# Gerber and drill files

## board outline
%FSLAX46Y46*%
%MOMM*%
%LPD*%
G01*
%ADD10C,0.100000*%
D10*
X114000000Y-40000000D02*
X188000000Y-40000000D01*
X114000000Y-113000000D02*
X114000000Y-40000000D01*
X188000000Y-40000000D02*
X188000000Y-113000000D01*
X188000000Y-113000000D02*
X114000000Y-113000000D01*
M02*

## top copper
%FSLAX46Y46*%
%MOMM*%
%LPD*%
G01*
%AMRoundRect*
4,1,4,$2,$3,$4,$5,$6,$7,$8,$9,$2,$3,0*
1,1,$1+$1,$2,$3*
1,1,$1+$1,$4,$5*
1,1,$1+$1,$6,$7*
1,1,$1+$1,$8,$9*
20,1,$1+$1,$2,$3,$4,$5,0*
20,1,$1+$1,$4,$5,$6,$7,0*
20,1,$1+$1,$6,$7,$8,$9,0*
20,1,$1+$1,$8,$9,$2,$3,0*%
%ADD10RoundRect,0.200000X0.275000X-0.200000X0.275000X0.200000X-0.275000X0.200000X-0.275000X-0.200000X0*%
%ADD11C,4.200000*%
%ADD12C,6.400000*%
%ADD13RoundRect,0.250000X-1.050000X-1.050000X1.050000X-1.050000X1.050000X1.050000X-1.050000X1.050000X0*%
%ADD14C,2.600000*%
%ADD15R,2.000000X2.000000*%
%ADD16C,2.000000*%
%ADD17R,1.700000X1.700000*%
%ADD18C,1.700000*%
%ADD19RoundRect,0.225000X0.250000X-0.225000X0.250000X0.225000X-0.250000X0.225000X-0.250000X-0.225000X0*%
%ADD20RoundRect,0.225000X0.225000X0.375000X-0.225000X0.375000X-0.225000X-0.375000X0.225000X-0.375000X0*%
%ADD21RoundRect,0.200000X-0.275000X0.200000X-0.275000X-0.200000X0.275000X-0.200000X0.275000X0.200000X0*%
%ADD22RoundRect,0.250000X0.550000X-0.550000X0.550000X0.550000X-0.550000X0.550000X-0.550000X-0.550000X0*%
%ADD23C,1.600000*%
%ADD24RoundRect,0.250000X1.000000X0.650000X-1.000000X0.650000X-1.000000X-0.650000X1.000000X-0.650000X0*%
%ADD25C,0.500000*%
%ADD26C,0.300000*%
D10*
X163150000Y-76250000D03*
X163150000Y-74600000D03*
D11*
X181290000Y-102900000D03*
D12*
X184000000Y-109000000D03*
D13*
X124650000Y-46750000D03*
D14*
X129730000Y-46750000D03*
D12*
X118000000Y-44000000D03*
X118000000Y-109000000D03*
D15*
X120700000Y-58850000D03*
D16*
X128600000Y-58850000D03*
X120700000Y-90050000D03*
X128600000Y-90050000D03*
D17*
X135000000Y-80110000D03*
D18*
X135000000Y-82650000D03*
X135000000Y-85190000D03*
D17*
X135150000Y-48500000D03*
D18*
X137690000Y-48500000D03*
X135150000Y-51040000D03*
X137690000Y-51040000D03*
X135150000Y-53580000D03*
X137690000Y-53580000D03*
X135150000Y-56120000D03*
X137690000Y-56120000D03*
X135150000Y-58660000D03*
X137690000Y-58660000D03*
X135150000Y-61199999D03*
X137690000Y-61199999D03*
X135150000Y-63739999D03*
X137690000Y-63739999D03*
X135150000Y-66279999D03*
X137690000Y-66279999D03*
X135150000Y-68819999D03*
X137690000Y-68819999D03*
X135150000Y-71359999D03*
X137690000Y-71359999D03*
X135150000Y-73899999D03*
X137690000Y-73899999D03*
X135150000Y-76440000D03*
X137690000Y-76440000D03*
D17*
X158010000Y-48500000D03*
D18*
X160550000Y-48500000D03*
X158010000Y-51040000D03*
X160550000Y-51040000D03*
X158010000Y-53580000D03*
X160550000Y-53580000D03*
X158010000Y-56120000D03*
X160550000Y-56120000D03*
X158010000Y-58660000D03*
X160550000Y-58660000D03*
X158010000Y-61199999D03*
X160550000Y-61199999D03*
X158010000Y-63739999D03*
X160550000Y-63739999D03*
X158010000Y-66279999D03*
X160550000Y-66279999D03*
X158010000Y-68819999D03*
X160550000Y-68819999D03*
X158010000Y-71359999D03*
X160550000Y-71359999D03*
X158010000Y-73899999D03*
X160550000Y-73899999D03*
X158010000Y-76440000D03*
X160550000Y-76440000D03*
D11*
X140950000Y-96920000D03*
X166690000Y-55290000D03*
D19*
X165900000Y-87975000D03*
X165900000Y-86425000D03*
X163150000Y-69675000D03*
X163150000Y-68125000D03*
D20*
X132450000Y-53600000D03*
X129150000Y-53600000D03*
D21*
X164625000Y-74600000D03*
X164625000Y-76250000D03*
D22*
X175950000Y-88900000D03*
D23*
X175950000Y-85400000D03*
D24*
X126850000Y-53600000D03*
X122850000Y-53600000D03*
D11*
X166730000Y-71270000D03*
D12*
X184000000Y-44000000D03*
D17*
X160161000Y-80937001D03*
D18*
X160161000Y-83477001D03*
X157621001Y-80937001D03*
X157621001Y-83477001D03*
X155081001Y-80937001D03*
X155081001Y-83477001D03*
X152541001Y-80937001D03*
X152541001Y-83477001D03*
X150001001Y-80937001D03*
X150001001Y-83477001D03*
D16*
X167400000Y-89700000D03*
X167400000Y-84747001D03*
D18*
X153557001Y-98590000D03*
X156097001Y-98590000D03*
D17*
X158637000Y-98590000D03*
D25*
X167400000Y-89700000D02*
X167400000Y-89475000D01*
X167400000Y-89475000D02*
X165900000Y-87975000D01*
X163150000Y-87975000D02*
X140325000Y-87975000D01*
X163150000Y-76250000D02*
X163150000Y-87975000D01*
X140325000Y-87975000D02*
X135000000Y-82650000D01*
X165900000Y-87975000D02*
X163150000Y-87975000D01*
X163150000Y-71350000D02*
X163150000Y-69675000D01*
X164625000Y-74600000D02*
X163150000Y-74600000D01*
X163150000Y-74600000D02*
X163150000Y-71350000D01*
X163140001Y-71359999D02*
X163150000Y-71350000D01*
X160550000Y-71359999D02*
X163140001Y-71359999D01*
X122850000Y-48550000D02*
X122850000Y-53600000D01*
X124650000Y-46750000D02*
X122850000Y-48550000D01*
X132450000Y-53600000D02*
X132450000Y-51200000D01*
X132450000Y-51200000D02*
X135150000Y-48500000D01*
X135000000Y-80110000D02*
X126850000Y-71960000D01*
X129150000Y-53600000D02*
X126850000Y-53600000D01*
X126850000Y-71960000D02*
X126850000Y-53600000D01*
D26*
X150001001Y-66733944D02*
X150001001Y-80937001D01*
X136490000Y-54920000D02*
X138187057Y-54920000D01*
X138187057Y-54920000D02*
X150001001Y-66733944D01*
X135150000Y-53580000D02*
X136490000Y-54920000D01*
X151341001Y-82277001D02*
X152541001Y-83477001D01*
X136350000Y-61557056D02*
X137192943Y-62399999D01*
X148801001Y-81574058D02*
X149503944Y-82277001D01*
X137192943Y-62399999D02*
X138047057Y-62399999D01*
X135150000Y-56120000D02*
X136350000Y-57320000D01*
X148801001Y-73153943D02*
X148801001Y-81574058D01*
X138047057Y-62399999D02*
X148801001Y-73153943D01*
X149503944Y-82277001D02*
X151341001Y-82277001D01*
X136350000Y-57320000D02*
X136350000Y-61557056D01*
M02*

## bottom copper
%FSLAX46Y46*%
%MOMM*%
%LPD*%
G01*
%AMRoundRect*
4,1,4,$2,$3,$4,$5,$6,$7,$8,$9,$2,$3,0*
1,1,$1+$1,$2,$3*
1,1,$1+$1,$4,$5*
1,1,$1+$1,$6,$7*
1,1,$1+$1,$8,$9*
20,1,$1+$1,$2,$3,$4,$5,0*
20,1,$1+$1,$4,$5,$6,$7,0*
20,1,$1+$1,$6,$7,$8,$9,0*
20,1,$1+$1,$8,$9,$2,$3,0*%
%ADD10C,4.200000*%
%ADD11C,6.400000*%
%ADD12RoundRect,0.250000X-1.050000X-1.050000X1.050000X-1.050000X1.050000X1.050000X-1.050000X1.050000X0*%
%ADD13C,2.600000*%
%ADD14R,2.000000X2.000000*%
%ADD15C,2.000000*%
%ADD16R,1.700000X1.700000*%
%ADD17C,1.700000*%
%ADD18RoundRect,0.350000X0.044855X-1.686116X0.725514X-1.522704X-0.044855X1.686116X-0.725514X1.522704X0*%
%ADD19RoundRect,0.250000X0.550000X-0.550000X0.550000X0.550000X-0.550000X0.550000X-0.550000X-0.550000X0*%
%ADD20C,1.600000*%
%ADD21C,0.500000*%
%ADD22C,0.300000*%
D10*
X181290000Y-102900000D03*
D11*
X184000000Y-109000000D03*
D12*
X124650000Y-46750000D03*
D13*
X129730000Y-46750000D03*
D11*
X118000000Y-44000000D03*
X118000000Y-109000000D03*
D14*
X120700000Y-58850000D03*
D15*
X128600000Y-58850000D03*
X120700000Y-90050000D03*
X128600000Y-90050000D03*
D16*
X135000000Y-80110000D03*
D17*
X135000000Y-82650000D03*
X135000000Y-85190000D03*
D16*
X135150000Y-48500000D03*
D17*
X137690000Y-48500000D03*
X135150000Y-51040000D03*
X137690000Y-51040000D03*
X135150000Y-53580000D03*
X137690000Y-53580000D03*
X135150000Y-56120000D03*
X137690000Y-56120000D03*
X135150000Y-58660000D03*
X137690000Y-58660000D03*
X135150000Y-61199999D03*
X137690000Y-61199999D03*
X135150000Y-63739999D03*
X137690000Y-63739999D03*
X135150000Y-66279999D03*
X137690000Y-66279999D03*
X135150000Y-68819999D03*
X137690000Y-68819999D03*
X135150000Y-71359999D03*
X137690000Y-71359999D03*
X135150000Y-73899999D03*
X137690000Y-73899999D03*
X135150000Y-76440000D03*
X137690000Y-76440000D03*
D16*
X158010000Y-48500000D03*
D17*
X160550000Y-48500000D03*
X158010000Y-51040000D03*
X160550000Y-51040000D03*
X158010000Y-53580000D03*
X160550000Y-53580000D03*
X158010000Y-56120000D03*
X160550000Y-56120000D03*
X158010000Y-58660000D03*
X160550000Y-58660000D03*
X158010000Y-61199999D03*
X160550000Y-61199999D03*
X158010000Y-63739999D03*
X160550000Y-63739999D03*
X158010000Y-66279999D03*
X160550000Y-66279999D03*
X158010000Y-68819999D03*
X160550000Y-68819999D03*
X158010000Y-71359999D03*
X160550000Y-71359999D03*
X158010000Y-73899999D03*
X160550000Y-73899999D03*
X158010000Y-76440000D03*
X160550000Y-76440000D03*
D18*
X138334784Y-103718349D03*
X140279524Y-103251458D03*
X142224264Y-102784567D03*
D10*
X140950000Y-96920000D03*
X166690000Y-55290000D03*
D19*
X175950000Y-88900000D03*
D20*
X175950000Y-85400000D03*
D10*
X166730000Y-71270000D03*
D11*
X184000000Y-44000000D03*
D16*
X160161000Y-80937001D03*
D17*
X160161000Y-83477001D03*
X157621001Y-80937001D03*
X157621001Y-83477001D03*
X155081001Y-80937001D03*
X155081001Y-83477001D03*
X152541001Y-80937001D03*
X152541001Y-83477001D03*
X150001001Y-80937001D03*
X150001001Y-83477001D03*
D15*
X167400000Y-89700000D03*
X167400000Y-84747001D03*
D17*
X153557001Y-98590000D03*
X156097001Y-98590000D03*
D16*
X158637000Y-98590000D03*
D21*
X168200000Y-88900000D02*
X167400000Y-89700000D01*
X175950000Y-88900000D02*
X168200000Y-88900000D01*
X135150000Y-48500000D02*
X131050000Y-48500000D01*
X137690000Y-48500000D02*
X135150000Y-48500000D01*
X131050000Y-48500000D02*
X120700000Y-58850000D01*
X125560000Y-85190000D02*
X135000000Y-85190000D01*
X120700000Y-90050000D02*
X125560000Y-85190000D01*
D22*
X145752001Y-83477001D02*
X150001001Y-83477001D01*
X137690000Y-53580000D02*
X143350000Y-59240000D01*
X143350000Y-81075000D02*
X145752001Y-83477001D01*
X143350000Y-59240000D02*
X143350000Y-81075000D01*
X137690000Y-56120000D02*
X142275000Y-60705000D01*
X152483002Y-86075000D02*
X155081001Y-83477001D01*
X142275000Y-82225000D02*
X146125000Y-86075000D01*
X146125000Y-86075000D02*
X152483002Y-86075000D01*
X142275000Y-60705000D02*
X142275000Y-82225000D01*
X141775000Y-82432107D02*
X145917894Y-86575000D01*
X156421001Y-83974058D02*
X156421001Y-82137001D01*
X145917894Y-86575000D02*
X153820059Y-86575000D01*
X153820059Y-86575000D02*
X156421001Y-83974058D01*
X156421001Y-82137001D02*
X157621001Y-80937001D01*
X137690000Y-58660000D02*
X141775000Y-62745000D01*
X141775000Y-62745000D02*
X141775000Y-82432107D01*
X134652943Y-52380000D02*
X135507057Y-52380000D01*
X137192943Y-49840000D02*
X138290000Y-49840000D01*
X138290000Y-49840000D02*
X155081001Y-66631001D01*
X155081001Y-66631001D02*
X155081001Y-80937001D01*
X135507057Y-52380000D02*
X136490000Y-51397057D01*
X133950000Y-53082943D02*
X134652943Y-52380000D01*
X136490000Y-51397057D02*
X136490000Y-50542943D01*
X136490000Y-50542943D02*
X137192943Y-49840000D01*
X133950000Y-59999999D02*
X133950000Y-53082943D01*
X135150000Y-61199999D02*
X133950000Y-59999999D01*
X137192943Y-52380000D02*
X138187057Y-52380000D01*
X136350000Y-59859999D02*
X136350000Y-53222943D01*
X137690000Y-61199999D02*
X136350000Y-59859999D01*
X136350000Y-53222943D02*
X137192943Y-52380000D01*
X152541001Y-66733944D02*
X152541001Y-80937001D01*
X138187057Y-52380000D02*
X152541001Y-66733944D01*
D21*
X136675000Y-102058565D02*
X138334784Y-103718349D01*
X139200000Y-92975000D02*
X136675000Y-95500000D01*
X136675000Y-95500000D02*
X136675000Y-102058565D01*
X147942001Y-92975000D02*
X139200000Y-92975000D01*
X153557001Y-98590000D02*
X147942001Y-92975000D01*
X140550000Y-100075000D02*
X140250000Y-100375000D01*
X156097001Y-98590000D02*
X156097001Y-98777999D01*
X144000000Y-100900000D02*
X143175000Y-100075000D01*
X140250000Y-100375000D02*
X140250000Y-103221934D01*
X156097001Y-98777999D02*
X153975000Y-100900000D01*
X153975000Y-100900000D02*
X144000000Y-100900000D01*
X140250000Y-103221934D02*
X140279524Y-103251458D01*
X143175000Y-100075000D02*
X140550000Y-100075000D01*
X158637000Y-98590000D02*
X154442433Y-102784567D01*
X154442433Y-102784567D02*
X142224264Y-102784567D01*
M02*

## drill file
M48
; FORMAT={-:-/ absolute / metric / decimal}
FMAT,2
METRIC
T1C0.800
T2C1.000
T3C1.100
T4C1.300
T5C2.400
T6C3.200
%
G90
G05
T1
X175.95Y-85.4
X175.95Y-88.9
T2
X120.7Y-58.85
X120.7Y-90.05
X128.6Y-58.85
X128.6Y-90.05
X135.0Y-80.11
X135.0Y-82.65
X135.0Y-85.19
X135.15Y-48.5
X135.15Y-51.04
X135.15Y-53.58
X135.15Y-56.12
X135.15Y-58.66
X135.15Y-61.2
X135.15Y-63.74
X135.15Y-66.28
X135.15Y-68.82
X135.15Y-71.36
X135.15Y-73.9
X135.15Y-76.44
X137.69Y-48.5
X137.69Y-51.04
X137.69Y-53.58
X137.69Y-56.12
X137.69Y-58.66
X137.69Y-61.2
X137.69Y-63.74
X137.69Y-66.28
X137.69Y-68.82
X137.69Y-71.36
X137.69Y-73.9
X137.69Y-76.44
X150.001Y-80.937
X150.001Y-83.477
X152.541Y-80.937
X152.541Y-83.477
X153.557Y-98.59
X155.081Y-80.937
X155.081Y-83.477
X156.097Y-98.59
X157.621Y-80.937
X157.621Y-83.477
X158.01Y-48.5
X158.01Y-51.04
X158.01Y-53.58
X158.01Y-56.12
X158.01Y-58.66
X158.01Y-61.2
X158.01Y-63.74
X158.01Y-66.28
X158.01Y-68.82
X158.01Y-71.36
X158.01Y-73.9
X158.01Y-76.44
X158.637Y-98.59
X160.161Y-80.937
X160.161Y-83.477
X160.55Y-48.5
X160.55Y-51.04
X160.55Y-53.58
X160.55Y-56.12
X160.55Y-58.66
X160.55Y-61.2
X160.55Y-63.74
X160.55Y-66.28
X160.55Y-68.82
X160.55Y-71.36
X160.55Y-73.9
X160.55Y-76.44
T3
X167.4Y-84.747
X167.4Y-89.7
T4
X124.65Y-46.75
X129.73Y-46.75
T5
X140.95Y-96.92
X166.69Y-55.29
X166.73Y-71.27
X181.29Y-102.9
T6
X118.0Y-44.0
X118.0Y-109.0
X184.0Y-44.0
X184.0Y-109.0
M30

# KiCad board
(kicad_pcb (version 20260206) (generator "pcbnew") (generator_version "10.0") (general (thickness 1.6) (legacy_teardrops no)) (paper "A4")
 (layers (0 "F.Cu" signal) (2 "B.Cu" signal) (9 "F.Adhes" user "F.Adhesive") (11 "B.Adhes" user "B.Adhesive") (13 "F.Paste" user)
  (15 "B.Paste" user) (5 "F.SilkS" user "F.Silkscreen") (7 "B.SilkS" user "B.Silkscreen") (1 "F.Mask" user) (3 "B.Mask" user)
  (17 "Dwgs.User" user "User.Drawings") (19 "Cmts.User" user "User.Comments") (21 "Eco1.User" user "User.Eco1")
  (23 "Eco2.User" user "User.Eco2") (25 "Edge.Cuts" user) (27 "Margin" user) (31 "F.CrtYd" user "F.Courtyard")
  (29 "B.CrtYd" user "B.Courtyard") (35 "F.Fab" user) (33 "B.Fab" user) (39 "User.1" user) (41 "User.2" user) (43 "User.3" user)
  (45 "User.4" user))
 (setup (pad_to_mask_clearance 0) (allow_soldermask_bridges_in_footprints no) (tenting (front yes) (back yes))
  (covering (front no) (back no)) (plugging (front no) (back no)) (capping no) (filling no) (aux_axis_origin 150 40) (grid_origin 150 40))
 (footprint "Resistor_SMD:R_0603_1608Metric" (layer "F.Cu") (at 163.15 75.425 90)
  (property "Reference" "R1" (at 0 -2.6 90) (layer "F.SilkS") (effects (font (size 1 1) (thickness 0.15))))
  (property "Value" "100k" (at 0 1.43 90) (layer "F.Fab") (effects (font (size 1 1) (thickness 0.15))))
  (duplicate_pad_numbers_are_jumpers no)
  (pad "1" smd roundrect (at -0.825 0 90) (size 0.8 0.95) (layers "F.Cu" "F.Mask" "F.Paste") (roundrect_rratio 0.25) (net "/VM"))
  (pad "2" smd roundrect (at 0.825 0 90) (size 0.8 0.95) (layers "F.Cu" "F.Mask" "F.Paste") (roundrect_rratio 0.25) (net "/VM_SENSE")))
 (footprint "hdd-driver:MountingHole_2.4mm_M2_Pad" (layer "F.Cu") (at 181.29 102.9)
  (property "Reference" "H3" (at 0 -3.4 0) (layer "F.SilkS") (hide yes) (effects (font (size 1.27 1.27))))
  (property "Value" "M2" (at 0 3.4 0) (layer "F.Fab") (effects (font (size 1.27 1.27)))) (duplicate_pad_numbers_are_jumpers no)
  (pad "1" thru_hole circle (at 0 0) (size 4.2 4.2) (drill 2.4) (layers "*.Cu" "*.Mask") (remove_unused_layers no) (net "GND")))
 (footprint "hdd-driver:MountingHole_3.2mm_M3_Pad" (layer "F.Cu") (at 184 109)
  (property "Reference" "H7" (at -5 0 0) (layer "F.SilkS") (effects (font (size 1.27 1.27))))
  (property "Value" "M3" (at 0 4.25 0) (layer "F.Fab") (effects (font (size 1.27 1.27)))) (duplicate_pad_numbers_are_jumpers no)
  (pad "1" thru_hole circle (at 0 0) (size 6.4 6.4) (drill 3.2) (layers "*.Cu" "*.Mask") (remove_unused_layers no) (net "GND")))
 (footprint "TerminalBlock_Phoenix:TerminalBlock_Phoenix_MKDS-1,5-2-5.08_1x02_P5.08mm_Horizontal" (layer "F.Cu") (at 124.65 46.75)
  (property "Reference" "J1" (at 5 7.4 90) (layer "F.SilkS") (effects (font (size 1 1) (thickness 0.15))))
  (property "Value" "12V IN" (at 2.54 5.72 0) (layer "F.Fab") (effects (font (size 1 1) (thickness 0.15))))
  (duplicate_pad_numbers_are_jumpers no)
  (pad "1" thru_hole roundrect (at 0 0) (size 2.6 2.6) (drill 1.3) (layers "*.Cu" "*.Mask") (remove_unused_layers no)
   (roundrect_rratio 0.096154) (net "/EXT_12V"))
  (pad "2" thru_hole circle (at 5.08 0) (size 2.6 2.6) (drill 1.3) (layers "*.Cu" "*.Mask") (remove_unused_layers no) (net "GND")))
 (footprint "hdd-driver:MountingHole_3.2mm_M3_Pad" (layer "F.Cu") (at 118 44)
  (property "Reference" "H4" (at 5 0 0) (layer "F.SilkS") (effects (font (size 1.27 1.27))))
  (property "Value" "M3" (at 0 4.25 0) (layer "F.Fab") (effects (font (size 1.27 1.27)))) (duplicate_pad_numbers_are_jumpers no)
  (pad "1" thru_hole circle (at 0 0) (size 6.4 6.4) (drill 3.2) (layers "*.Cu" "*.Mask") (remove_unused_layers no) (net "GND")))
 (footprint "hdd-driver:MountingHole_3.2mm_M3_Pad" (layer "F.Cu") (at 118 109)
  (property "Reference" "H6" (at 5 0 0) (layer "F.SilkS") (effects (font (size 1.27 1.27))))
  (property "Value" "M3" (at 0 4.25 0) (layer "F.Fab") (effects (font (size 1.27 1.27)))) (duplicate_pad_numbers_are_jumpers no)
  (pad "1" thru_hole circle (at 0 0) (size 6.4 6.4) (drill 3.2) (layers "*.Cu" "*.Mask") (remove_unused_layers no) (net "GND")))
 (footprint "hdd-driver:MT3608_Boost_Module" (layer "F.Cu") (at 124.1 74.45 -90)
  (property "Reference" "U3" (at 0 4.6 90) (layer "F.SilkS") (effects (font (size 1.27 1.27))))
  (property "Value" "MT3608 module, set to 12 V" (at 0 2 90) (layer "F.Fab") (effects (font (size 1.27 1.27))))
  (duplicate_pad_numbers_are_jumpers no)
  (pad "1" thru_hole rect (at -15.6 3.4 270) (size 2 2) (drill 1) (layers "*.Cu" "*.Mask") (remove_unused_layers no) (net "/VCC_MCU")
   (thermal_bridge_angle 45))
  (pad "2" thru_hole circle (at -15.6 -4.5 270) (size 2 2) (drill 1) (layers "*.Cu" "*.Mask") (remove_unused_layers no) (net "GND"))
  (pad "3" thru_hole circle (at 15.6 3.4 270) (size 2 2) (drill 1) (layers "*.Cu" "*.Mask") (remove_unused_layers no) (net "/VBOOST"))
  (pad "4" thru_hole circle (at 15.6 -4.5 270) (size 2 2) (drill 1) (layers "*.Cu" "*.Mask") (remove_unused_layers no) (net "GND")))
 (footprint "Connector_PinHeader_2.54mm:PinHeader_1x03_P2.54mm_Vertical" (layer "F.Cu") (at 135 80.11)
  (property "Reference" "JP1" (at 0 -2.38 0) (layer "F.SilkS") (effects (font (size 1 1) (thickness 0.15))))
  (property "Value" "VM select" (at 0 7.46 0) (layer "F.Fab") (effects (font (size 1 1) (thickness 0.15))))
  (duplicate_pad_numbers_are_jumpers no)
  (pad "1" thru_hole rect (at 0 0) (size 1.7 1.7) (drill 1) (layers "*.Cu" "*.Mask") (remove_unused_layers no) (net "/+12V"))
  (pad "2" thru_hole circle (at 0 2.54) (size 1.7 1.7) (drill 1) (layers "*.Cu" "*.Mask") (remove_unused_layers no) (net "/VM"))
  (pad "3" thru_hole circle (at 0 5.08) (size 1.7 1.7) (drill 1) (layers "*.Cu" "*.Mask") (remove_unused_layers no) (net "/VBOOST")))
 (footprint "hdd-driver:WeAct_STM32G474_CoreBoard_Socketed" (layer "F.Cu") (at 147.85 59.67 -90)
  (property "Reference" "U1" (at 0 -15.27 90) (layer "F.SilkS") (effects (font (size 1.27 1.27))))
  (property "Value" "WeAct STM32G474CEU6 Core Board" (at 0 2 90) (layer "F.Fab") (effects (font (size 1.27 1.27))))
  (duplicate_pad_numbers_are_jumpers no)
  (pad "P1.1" thru_hole rect (at -11.17 12.7 270) (size 1.7 1.7) (drill 1) (layers "*.Cu" "*.Mask") (remove_unused_layers no)
   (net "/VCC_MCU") (thermal_bridge_angle 45))
  (pad "P1.2" thru_hole circle (at -11.17 10.16 270) (size 1.7 1.7) (drill 1) (layers "*.Cu" "*.Mask") (remove_unused_layers no)
   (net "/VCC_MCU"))
  (pad "P1.3" thru_hole circle (at -8.63 12.7 270) (size 1.7 1.7) (drill 1) (layers "*.Cu" "*.Mask") (remove_unused_layers no) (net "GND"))
  (pad "P1.4" thru_hole circle (at -8.63 10.16 270) (size 1.7 1.7) (drill 1) (layers "*.Cu" "*.Mask") (remove_unused_layers no) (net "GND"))
  (pad "P1.5" thru_hole circle (at -6.09 12.7 270) (size 1.7 1.7) (drill 1) (layers "*.Cu" "*.Mask") (remove_unused_layers no)
   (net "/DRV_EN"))
  (pad "P1.6" thru_hole circle (at -6.09 10.16 270) (size 1.7 1.7) (drill 1) (layers "*.Cu" "*.Mask") (remove_unused_layers no)
   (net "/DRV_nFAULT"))
  (pad "P1.7" thru_hole circle (at -3.55 12.7 270) (size 1.7 1.7) (drill 1) (layers "*.Cu" "*.Mask") (remove_unused_layers no)
   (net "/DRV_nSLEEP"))
  (pad "P1.8" thru_hole circle (at -3.55 10.16 270) (size 1.7 1.7) (drill 1) (layers "*.Cu" "*.Mask") (remove_unused_layers no)
   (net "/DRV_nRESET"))
  (pad "P1.9" thru_hole circle (at -1.01 12.7 270) (size 1.7 1.7) (drill 1) (layers "*.Cu" "*.Mask") (remove_unused_layers no)
   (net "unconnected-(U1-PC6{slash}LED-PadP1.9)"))
  (pad "P1.10" thru_hole circle (at -1.01 10.16 270) (size 1.7 1.7) (drill 1) (layers "*.Cu" "*.Mask") (remove_unused_layers no)
   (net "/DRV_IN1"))
  (pad "P1.11" thru_hole circle (at 1.529999 12.7 270) (size 1.7 1.7) (drill 1) (layers "*.Cu" "*.Mask") (remove_unused_layers no)
   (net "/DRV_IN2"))
  (pad "P1.12" thru_hole circle (at 1.529999 10.16 270) (size 1.7 1.7) (drill 1) (layers "*.Cu" "*.Mask") (remove_unused_layers no)
   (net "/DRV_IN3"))
  (pad "P1.13" thru_hole circle (at 4.069999 12.7 270) (size 1.7 1.7) (drill 1) (layers "*.Cu" "*.Mask") (remove_unused_layers no)
   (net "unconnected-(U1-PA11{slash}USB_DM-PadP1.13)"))
  (pad "P1.14" thru_hole circle (at 4.069999 10.16 270) (size 1.7 1.7) (drill 1) (layers "*.Cu" "*.Mask") (remove_unused_layers no)
   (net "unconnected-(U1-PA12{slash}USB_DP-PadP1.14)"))
  (pad "P1.15" thru_hole circle (at 6.609999 12.7 270) (size 1.7 1.7) (drill 1) (layers "*.Cu" "*.Mask") (remove_unused_layers no)
   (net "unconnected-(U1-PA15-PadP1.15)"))
  (pad "P1.16" thru_hole circle (at 6.609999 10.16 270) (size 1.7 1.7) (drill 1) (layers "*.Cu" "*.Mask") (remove_unused_layers no)
   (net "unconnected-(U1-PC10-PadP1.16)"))
  (pad "P1.17" thru_hole circle (at 9.149999 12.7 270) (size 1.7 1.7) (drill 1) (layers "*.Cu" "*.Mask") (remove_unused_layers no)
   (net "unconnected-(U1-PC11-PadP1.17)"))
  (pad "P1.18" thru_hole circle (at 9.149999 10.16 270) (size 1.7 1.7) (drill 1) (layers "*.Cu" "*.Mask") (remove_unused_layers no)
   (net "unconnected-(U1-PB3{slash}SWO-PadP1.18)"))
  (pad "P1.19" thru_hole circle (at 11.689999 12.7 270) (size 1.7 1.7) (drill 1) (layers "*.Cu" "*.Mask") (remove_unused_layers no)
   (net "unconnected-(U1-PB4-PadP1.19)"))
  (pad "P1.20" thru_hole circle (at 11.689999 10.16 270) (size 1.7 1.7) (drill 1) (layers "*.Cu" "*.Mask") (remove_unused_layers no)
   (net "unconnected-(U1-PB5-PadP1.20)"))
  (pad "P1.21" thru_hole circle (at 14.229999 12.7 270) (size 1.7 1.7) (drill 1) (layers "*.Cu" "*.Mask") (remove_unused_layers no)
   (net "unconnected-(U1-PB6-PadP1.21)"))
  (pad "P1.22" thru_hole circle (at 14.229999 10.16 270) (size 1.7 1.7) (drill 1) (layers "*.Cu" "*.Mask") (remove_unused_layers no)
   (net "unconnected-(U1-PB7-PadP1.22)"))
  (pad "P1.23" thru_hole circle (at 16.77 12.7 270) (size 1.7 1.7) (drill 1) (layers "*.Cu" "*.Mask") (remove_unused_layers no)
   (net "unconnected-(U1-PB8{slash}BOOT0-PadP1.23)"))
  (pad "P1.24" thru_hole circle (at 16.77 10.16 270) (size 1.7 1.7) (drill 1) (layers "*.Cu" "*.Mask") (remove_unused_layers no)
   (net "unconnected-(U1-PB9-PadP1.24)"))
  (pad "P2.1" thru_hole rect (at -11.17 -10.16 270) (size 1.7 1.7) (drill 1) (layers "*.Cu" "*.Mask") (remove_unused_layers no)
   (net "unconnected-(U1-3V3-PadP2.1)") (thermal_bridge_angle 45))
  (pad "P2.2" thru_hole circle (at -11.17 -12.7 270) (size 1.7 1.7) (drill 1) (layers "*.Cu" "*.Mask") (remove_unused_layers no)
   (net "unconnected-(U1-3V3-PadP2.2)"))
  (pad "P2.3" thru_hole circle (at -8.63 -10.16 270) (size 1.7 1.7) (drill 1) (layers "*.Cu" "*.Mask") (remove_unused_layers no) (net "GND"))
  (pad "P2.4" thru_hole circle (at -8.63 -12.7 270) (size 1.7 1.7) (drill 1) (layers "*.Cu" "*.Mask") (remove_unused_layers no) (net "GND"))
  (pad "P2.5" thru_hole circle (at -6.09 -10.16 270) (size 1.7 1.7) (drill 1) (layers "*.Cu" "*.Mask") (remove_unused_layers no)
   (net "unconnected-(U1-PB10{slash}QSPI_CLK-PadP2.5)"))
  (pad "P2.6" thru_hole circle (at -6.09 -12.7 270) (size 1.7 1.7) (drill 1) (layers "*.Cu" "*.Mask") (remove_unused_layers no)
   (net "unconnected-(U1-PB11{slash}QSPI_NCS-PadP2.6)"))
  (pad "P2.7" thru_hole circle (at -3.55 -10.16 270) (size 1.7 1.7) (drill 1) (layers "*.Cu" "*.Mask") (remove_unused_layers no)
   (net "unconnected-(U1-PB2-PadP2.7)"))
  (pad "P2.8" thru_hole circle (at -3.55 -12.7 270) (size 1.7 1.7) (drill 1) (layers "*.Cu" "*.Mask") (remove_unused_layers no)
   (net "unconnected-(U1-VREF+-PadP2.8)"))
  (pad "P2.9" thru_hole circle (at -1.01 -10.16 270) (size 1.7 1.7) (drill 1) (layers "*.Cu" "*.Mask") (remove_unused_layers no)
   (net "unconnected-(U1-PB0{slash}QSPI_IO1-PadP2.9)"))
  (pad "P2.10" thru_hole circle (at -1.01 -12.7 270) (size 1.7 1.7) (drill 1) (layers "*.Cu" "*.Mask") (remove_unused_layers no)
   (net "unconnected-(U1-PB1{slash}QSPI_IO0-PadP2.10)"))
  (pad "P2.11" thru_hole circle (at 1.529999 -10.16 270) (size 1.7 1.7) (drill 1) (layers "*.Cu" "*.Mask") (remove_unused_layers no)
   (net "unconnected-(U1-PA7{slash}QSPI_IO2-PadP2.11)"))
  (pad "P2.12" thru_hole circle (at 1.529999 -12.7 270) (size 1.7 1.7) (drill 1) (layers "*.Cu" "*.Mask") (remove_unused_layers no)
   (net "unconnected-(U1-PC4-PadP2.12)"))
  (pad "P2.13" thru_hole circle (at 4.069999 -10.16 270) (size 1.7 1.7) (drill 1) (layers "*.Cu" "*.Mask") (remove_unused_layers no)
   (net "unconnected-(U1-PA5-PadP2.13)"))
  (pad "P2.14" thru_hole circle (at 4.069999 -12.7 270) (size 1.7 1.7) (drill 1) (layers "*.Cu" "*.Mask") (remove_unused_layers no)
   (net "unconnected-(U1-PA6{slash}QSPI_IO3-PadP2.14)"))
  (pad "P2.15" thru_hole circle (at 6.609999 -10.16 270) (size 1.7 1.7) (drill 1) (layers "*.Cu" "*.Mask") (remove_unused_layers no)
   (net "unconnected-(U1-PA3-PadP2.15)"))
  (pad "P2.16" thru_hole circle (at 6.609999 -12.7 270) (size 1.7 1.7) (drill 1) (layers "*.Cu" "*.Mask") (remove_unused_layers no)
   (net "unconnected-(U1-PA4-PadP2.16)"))
  (pad "P2.17" thru_hole circle (at 9.149999 -10.16 270) (size 1.7 1.7) (drill 1) (layers "*.Cu" "*.Mask") (remove_unused_layers no)
   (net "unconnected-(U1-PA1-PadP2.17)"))
  (pad "P2.18" thru_hole circle (at 9.149999 -12.7 270) (size 1.7 1.7) (drill 1) (layers "*.Cu" "*.Mask") (remove_unused_layers no)
   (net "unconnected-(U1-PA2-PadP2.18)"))
  (pad "P2.19" thru_hole circle (at 11.689999 -10.16 270) (size 1.7 1.7) (drill 1) (layers "*.Cu" "*.Mask") (remove_unused_layers no)
   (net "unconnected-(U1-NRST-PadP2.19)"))
  (pad "P2.20" thru_hole circle (at 11.689999 -12.7 270) (size 1.7 1.7) (drill 1) (layers "*.Cu" "*.Mask") (remove_unused_layers no)
   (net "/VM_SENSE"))
  (pad "P2.21" thru_hole circle (at 14.229999 -10.16 270) (size 1.7 1.7) (drill 1) (layers "*.Cu" "*.Mask") (remove_unused_layers no)
   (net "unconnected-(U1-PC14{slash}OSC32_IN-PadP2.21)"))
  (pad "P2.22" thru_hole circle (at 14.229999 -12.7 270) (size 1.7 1.7) (drill 1) (layers "*.Cu" "*.Mask") (remove_unused_layers no)
   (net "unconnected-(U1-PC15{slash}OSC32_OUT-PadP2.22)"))
  (pad "P2.23" thru_hole circle (at 16.77 -10.16 270) (size 1.7 1.7) (drill 1) (layers "*.Cu" "*.Mask") (remove_unused_layers no)
   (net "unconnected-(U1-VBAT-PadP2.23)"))
  (pad "P2.24" thru_hole circle (at 16.77 -12.7 270) (size 1.7 1.7) (drill 1) (layers "*.Cu" "*.Mask") (remove_unused_layers no)
   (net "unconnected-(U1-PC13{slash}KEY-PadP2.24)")))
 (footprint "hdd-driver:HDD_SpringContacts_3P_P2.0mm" (layer "F.Cu") (at 140.95 96.92 13.5)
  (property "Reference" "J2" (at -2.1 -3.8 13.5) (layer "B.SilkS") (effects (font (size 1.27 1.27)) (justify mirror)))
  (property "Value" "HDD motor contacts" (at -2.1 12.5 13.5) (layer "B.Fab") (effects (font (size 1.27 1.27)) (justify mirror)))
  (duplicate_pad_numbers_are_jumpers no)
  (pad "1" smd roundrect (at -4.13 6 13.5) (size 1.4 4) (layers "B.Cu" "B.Mask") (roundrect_rratio 0.25) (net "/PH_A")
   (thermal_bridge_angle 45))
  (pad "2" smd roundrect (at -2.13 6 13.5) (size 1.4 4) (layers "B.Cu" "B.Mask") (roundrect_rratio 0.25) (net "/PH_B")
   (thermal_bridge_angle 45))
  (pad "3" smd roundrect (at -0.13 6 13.5) (size 1.4 4) (layers "B.Cu" "B.Mask") (roundrect_rratio 0.25) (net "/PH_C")
   (thermal_bridge_angle 45))
  (pad "4" thru_hole circle (at 0 0 13.5) (size 4.2 4.2) (drill 2.4) (layers "*.Cu" "*.Mask") (remove_unused_layers no) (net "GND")))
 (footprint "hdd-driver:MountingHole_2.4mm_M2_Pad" (layer "F.Cu") (at 166.69 55.29)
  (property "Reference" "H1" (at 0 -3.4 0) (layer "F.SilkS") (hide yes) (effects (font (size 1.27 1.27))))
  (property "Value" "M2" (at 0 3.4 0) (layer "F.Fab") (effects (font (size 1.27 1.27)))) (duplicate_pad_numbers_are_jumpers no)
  (pad "1" thru_hole circle (at 0 0) (size 4.2 4.2) (drill 2.4) (layers "*.Cu" "*.Mask") (remove_unused_layers no) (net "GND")))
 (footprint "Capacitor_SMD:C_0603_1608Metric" (layer "F.Cu") (at 165.9 87.2 90)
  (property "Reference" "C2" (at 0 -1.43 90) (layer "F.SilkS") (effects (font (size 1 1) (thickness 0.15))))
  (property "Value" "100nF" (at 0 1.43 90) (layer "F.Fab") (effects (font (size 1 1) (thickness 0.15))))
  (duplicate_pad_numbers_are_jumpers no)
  (pad "1" smd roundrect (at -0.775 0 90) (size 0.9 0.95) (layers "F.Cu" "F.Mask" "F.Paste") (roundrect_rratio 0.25) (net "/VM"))
  (pad "2" smd roundrect (at 0.775 0 90) (size 0.9 0.95) (layers "F.Cu" "F.Mask" "F.Paste") (roundrect_rratio 0.25) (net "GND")))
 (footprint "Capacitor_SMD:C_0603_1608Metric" (layer "F.Cu") (at 163.15 68.9 90)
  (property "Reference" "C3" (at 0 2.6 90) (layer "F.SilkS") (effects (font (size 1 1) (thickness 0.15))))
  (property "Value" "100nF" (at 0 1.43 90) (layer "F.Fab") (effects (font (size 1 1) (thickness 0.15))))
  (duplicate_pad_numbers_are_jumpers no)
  (pad "1" smd roundrect (at -0.775 0 90) (size 0.9 0.95) (layers "F.Cu" "F.Mask" "F.Paste") (roundrect_rratio 0.25) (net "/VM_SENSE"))
  (pad "2" smd roundrect (at 0.775 0 90) (size 0.9 0.95) (layers "F.Cu" "F.Mask" "F.Paste") (roundrect_rratio 0.25) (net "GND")))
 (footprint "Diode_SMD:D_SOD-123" (layer "F.Cu") (at 130.8 53.6 180)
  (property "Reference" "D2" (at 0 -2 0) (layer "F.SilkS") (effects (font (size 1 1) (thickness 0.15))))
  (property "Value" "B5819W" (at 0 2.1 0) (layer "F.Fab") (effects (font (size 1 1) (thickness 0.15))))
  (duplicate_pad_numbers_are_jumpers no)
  (pad "1" smd roundrect (at -1.65 0 180) (size 0.9 1.2) (layers "F.Cu" "F.Mask" "F.Paste") (roundrect_rratio 0.25) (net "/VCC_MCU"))
  (pad "2" smd roundrect (at 1.65 0 180) (size 0.9 1.2) (layers "F.Cu" "F.Mask" "F.Paste") (roundrect_rratio 0.25) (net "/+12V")))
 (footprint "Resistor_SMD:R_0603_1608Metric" (layer "F.Cu") (at 164.625 75.425 -90)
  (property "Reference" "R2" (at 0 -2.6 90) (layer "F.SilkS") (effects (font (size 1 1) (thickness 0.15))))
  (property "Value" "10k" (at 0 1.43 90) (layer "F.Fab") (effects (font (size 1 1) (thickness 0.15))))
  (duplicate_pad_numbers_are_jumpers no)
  (pad "1" smd roundrect (at -0.825 0 270) (size 0.8 0.95) (layers "F.Cu" "F.Mask" "F.Paste") (roundrect_rratio 0.25) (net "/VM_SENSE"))
  (pad "2" smd roundrect (at 0.825 0 270) (size 0.8 0.95) (layers "F.Cu" "F.Mask" "F.Paste") (roundrect_rratio 0.25) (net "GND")))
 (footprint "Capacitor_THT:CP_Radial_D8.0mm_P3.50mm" (layer "F.Cu") (at 175.95 88.9 90)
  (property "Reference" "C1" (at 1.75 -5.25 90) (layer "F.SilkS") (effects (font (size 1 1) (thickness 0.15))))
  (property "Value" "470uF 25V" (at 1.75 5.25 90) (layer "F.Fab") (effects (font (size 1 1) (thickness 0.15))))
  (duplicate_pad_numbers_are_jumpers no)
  (pad "1" thru_hole roundrect (at 0 0 90) (size 1.6 1.6) (drill 0.8) (layers "*.Cu" "*.Mask") (remove_unused_layers no)
   (roundrect_rratio 0.15625) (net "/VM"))
  (pad "2" thru_hole circle (at 3.5 0 90) (size 1.6 1.6) (drill 0.8) (layers "*.Cu" "*.Mask") (remove_unused_layers no) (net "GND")))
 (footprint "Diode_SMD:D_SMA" (layer "F.Cu") (at 124.85 53.6 180)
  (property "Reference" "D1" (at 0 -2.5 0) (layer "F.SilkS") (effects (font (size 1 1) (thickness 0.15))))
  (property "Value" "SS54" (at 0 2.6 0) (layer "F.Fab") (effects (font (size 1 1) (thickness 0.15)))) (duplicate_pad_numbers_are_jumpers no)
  (pad "1" smd roundrect (at -2 0 180) (size 2.5 1.8) (layers "F.Cu" "F.Mask" "F.Paste") (roundrect_rratio 0.1388888889) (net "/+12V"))
  (pad "2" smd roundrect (at 2 0 180) (size 2.5 1.8) (layers "F.Cu" "F.Mask" "F.Paste") (roundrect_rratio 0.1388888889) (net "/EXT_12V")))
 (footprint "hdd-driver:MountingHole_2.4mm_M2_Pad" (layer "F.Cu") (at 166.73 71.27)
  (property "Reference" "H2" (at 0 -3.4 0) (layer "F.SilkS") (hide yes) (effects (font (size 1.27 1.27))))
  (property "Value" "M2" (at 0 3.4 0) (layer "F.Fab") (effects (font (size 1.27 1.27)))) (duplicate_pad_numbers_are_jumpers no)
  (pad "1" thru_hole circle (at 0 0) (size 4.2 4.2) (drill 2.4) (layers "*.Cu" "*.Mask") (remove_unused_layers no) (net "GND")))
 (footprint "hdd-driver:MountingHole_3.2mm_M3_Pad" (layer "F.Cu") (at 184 44)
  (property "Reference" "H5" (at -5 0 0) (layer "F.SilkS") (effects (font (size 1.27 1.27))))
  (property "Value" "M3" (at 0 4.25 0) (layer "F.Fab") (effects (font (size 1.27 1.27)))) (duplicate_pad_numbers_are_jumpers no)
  (pad "1" thru_hole circle (at 0 0) (size 6.4 6.4) (drill 3.2) (layers "*.Cu" "*.Mask") (remove_unused_layers no) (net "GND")))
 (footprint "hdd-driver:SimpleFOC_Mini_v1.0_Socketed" (layer "F.Cu") (at 158.046017 89.491646)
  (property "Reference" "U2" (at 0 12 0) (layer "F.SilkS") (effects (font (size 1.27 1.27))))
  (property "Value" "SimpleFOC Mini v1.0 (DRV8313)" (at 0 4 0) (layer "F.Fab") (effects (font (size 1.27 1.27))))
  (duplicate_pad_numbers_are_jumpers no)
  (pad "1" thru_hole rect (at 2.114983 -8.554645) (size 1.7 1.7) (drill 1) (layers "*.Cu" "*.Mask") (remove_unused_layers no) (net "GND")
   (thermal_bridge_angle 45))
  (pad "2" thru_hole circle (at 2.114983 -6.014645) (size 1.7 1.7) (drill 1) (layers "*.Cu" "*.Mask") (remove_unused_layers no)
   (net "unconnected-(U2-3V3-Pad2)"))
  (pad "3" thru_hole circle (at -0.425016 -8.554645) (size 1.7 1.7) (drill 1) (layers "*.Cu" "*.Mask") (remove_unused_layers no)
   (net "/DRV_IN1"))
  (pad "4" thru_hole circle (at -0.425016 -6.014645) (size 1.7 1.7) (drill 1) (layers "*.Cu" "*.Mask") (remove_unused_layers no) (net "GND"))
  (pad "5" thru_hole circle (at -2.965016 -8.554645) (size 1.7 1.7) (drill 1) (layers "*.Cu" "*.Mask") (remove_unused_layers no)
   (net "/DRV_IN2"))
  (pad "6" thru_hole circle (at -2.965016 -6.014645) (size 1.7 1.7) (drill 1) (layers "*.Cu" "*.Mask") (remove_unused_layers no)
   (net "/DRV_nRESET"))
  (pad "7" thru_hole circle (at -5.505016 -8.554645) (size 1.7 1.7) (drill 1) (layers "*.Cu" "*.Mask") (remove_unused_layers no)
   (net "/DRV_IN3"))
  (pad "8" thru_hole circle (at -5.505016 -6.014645) (size 1.7 1.7) (drill 1) (layers "*.Cu" "*.Mask") (remove_unused_layers no)
   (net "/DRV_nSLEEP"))
  (pad "9" thru_hole circle (at -8.045016 -8.554645) (size 1.7 1.7) (drill 1) (layers "*.Cu" "*.Mask") (remove_unused_layers no)
   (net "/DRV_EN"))
  (pad "10" thru_hole circle (at -8.045016 -6.014645) (size 1.7 1.7) (drill 1) (layers "*.Cu" "*.Mask") (remove_unused_layers no)
   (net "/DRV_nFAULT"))
  (pad "11" thru_hole circle (at 9.353983 0.208354) (size 2 2) (drill 1.1) (layers "*.Cu" "*.Mask") (remove_unused_layers no) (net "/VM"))
  (pad "12" thru_hole circle (at 9.353983 -4.744645) (size 2 2) (drill 1.1) (layers "*.Cu" "*.Mask") (remove_unused_layers no) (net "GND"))
  (pad "13" thru_hole circle (at -4.489016 9.098354) (size 1.7 1.7) (drill 1) (layers "*.Cu" "*.Mask") (remove_unused_layers no)
   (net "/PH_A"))
  (pad "14" thru_hole circle (at -1.949016 9.098354) (size 1.7 1.7) (drill 1) (layers "*.Cu" "*.Mask") (remove_unused_layers no)
   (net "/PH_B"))
  (pad "15" thru_hole rect (at 0.590983 9.098354) (size 1.7 1.7) (drill 1) (layers "*.Cu" "*.Mask") (remove_unused_layers no) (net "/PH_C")
   (thermal_bridge_angle 45)))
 (gr_line (start 114 40) (end 188 40) (stroke (width 0.1) (type default)) (layer "Edge.Cuts"))
 (gr_line (start 114 113) (end 114 40) (stroke (width 0.1) (type default)) (layer "Edge.Cuts"))
 (gr_line (start 188 40) (end 188 113) (stroke (width 0.1) (type default)) (layer "Edge.Cuts"))
 (gr_line (start 188 113) (end 114 113) (stroke (width 0.1) (type default)) (layer "Edge.Cuts"))
 (segment (start 167.4 89.7) (end 167.4 89.475) (width 0.5) (layer "F.Cu") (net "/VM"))
 (segment (start 167.4 89.475) (end 165.9 87.975) (width 0.5) (layer "F.Cu") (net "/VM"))
 (segment (start 163.15 87.975) (end 140.325 87.975) (width 0.5) (layer "F.Cu") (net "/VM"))
 (segment (start 163.15 76.25) (end 163.15 87.975) (width 0.5) (layer "F.Cu") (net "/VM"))
 (segment (start 140.325 87.975) (end 135 82.65) (width 0.5) (layer "F.Cu") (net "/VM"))
 (segment (start 165.9 87.975) (end 163.15 87.975) (width 0.5) (layer "F.Cu") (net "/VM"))
 (segment (start 168.2 88.9) (end 167.4 89.7) (width 0.5) (layer "B.Cu") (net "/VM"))
 (segment (start 175.95 88.9) (end 168.2 88.9) (width 0.5) (layer "B.Cu") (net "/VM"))
 (segment (start 163.15 71.35) (end 163.15 69.675) (width 0.5) (layer "F.Cu") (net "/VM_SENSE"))
 (segment (start 164.625 74.6) (end 163.15 74.6) (width 0.5) (layer "F.Cu") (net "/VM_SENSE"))
 (segment (start 163.15 74.6) (end 163.15 71.35) (width 0.5) (layer "F.Cu") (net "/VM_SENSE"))
 (segment (start 163.140001 71.359999) (end 163.15 71.35) (width 0.5) (layer "F.Cu") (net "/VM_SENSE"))
 (segment (start 160.55 71.359999) (end 163.140001 71.359999) (width 0.5) (layer "F.Cu") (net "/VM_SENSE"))
 (segment (start 122.85 48.55) (end 122.85 53.6) (width 0.5) (layer "F.Cu") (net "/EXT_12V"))
 (segment (start 124.65 46.75) (end 122.85 48.55) (width 0.5) (layer "F.Cu") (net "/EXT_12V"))
 (segment (start 132.45 53.6) (end 132.45 51.2) (width 0.5) (layer "F.Cu") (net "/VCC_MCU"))
 (segment (start 132.45 51.2) (end 135.15 48.5) (width 0.5) (layer "F.Cu") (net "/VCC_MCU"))
 (segment (start 135.15 48.5) (end 131.05 48.5) (width 0.5) (layer "B.Cu") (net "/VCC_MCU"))
 (segment (start 137.69 48.5) (end 135.15 48.5) (width 0.5) (layer "B.Cu") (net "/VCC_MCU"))
 (segment (start 131.05 48.5) (end 120.7 58.85) (width 0.5) (layer "B.Cu") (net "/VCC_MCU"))
 (segment (start 125.56 85.19) (end 135 85.19) (width 0.5) (layer "B.Cu") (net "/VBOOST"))
 (segment (start 120.7 90.05) (end 125.56 85.19) (width 0.5) (layer "B.Cu") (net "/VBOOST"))
 (segment (start 135 80.11) (end 126.85 71.96) (width 0.5) (layer "F.Cu") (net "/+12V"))
 (segment (start 129.15 53.6) (end 126.85 53.6) (width 0.5) (layer "F.Cu") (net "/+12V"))
 (segment (start 126.85 71.96) (end 126.85 53.6) (width 0.5) (layer "F.Cu") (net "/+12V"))
 (segment (start 150.001001 66.733944) (end 150.001001 80.937001) (width 0.3) (layer "F.Cu") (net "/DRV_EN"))
 (segment (start 136.49 54.92) (end 138.187057 54.92) (width 0.3) (layer "F.Cu") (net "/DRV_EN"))
 (segment (start 138.187057 54.92) (end 150.001001 66.733944) (width 0.3) (layer "F.Cu") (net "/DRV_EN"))
 (segment (start 135.15 53.58) (end 136.49 54.92) (width 0.3) (layer "F.Cu") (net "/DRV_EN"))
 (segment (start 145.752001 83.477001) (end 150.001001 83.477001) (width 0.3) (layer "B.Cu") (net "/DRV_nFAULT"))
 (segment (start 137.69 53.58) (end 143.35 59.24) (width 0.3) (layer "B.Cu") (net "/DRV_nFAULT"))
 (segment (start 143.35 81.075) (end 145.752001 83.477001) (width 0.3) (layer "B.Cu") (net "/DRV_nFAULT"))
 (segment (start 143.35 59.24) (end 143.35 81.075) (width 0.3) (layer "B.Cu") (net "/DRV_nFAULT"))
 (segment (start 151.341001 82.277001) (end 152.541001 83.477001) (width 0.3) (layer "F.Cu") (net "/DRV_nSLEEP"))
 (segment (start 136.35 61.557056) (end 137.192943 62.399999) (width 0.3) (layer "F.Cu") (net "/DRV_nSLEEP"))
 (segment (start 148.801001 81.574058) (end 149.503944 82.277001) (width 0.3) (layer "F.Cu") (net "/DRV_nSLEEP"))
 (segment (start 137.192943 62.399999) (end 138.047057 62.399999) (width 0.3) (layer "F.Cu") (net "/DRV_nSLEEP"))
 (segment (start 135.15 56.12) (end 136.35 57.32) (width 0.3) (layer "F.Cu") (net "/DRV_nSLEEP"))
 (segment (start 148.801001 73.153943) (end 148.801001 81.574058) (width 0.3) (layer "F.Cu") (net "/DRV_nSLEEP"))
 (segment (start 138.047057 62.399999) (end 148.801001 73.153943) (width 0.3) (layer "F.Cu") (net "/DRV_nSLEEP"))
 (segment (start 149.503944 82.277001) (end 151.341001 82.277001) (width 0.3) (layer "F.Cu") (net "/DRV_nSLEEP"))
 (segment (start 136.35 57.32) (end 136.35 61.557056) (width 0.3) (layer "F.Cu") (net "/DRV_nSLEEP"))
 (segment (start 137.69 56.12) (end 142.275 60.705) (width 0.3) (layer "B.Cu") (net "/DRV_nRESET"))
 (segment (start 152.483002 86.075) (end 155.081001 83.477001) (width 0.3) (layer "B.Cu") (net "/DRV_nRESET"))
 (segment (start 142.275 82.225) (end 146.125 86.075) (width 0.3) (layer "B.Cu") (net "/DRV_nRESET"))
 (segment (start 146.125 86.075) (end 152.483002 86.075) (width 0.3) (layer "B.Cu") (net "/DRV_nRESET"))
 (segment (start 142.275 60.705) (end 142.275 82.225) (width 0.3) (layer "B.Cu") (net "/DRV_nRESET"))
 (segment (start 141.775 82.432107) (end 145.917894 86.575) (width 0.3) (layer "B.Cu") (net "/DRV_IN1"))
 (segment (start 156.421001 83.974058) (end 156.421001 82.137001) (width 0.3) (layer "B.Cu") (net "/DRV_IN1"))
 (segment (start 145.917894 86.575) (end 153.820059 86.575) (width 0.3) (layer "B.Cu") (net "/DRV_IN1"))
 (segment (start 153.820059 86.575) (end 156.421001 83.974058) (width 0.3) (layer "B.Cu") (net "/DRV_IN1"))
 (segment (start 156.421001 82.137001) (end 157.621001 80.937001) (width 0.3) (layer "B.Cu") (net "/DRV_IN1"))
 (segment (start 137.69 58.66) (end 141.775 62.745) (width 0.3) (layer "B.Cu") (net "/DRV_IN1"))
 (segment (start 141.775 62.745) (end 141.775 82.432107) (width 0.3) (layer "B.Cu") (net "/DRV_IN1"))
 (segment (start 134.652943 52.38) (end 135.507057 52.38) (width 0.3) (layer "B.Cu") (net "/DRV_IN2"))
 (segment (start 137.192943 49.84) (end 138.29 49.84) (width 0.3) (layer "B.Cu") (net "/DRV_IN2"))
 (segment (start 138.29 49.84) (end 155.081001 66.631001) (width 0.3) (layer "B.Cu") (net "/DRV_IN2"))
 (segment (start 155.081001 66.631001) (end 155.081001 80.937001) (width 0.3) (layer "B.Cu") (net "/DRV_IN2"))
 (segment (start 135.507057 52.38) (end 136.49 51.397057) (width 0.3) (layer "B.Cu") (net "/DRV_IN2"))
 (segment (start 133.95 53.082943) (end 134.652943 52.38) (width 0.3) (layer "B.Cu") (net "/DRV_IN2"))
 (segment (start 136.49 51.397057) (end 136.49 50.542943) (width 0.3) (layer "B.Cu") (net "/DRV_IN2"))
 (segment (start 136.49 50.542943) (end 137.192943 49.84) (width 0.3) (layer "B.Cu") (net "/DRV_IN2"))
 (segment (start 133.95 59.999999) (end 133.95 53.082943) (width 0.3) (layer "B.Cu") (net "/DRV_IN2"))
 (segment (start 135.15 61.199999) (end 133.95 59.999999) (width 0.3) (layer "B.Cu") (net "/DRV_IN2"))
 (segment (start 137.192943 52.38) (end 138.187057 52.38) (width 0.3) (layer "B.Cu") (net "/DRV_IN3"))
 (segment (start 136.35 59.859999) (end 136.35 53.222943) (width 0.3) (layer "B.Cu") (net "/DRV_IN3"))
 (segment (start 137.69 61.199999) (end 136.35 59.859999) (width 0.3) (layer "B.Cu") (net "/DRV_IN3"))
 (segment (start 136.35 53.222943) (end 137.192943 52.38) (width 0.3) (layer "B.Cu") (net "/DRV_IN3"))
 (segment (start 152.541001 66.733944) (end 152.541001 80.937001) (width 0.3) (layer "B.Cu") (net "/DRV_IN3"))
 (segment (start 138.187057 52.38) (end 152.541001 66.733944) (width 0.3) (layer "B.Cu") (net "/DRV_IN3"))
 (segment (start 136.675 102.058565) (end 138.334784 103.718349) (width 0.5) (layer "B.Cu") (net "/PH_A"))
 (segment (start 139.2 92.975) (end 136.675 95.5) (width 0.5) (layer "B.Cu") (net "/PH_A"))
 (segment (start 136.675 95.5) (end 136.675 102.058565) (width 0.5) (layer "B.Cu") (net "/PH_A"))
 (segment (start 147.942001 92.975) (end 139.2 92.975) (width 0.5) (layer "B.Cu") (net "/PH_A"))
 (segment (start 153.557001 98.59) (end 147.942001 92.975) (width 0.5) (layer "B.Cu") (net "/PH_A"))
 (segment (start 140.55 100.075) (end 140.25 100.375) (width 0.5) (layer "B.Cu") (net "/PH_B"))
 (segment (start 156.097001 98.59) (end 156.097001 98.777999) (width 0.5) (layer "B.Cu") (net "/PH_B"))
 (segment (start 144 100.9) (end 143.175 100.075) (width 0.5) (layer "B.Cu") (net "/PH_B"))
 (segment (start 140.25 100.375) (end 140.25 103.221934) (width 0.5) (layer "B.Cu") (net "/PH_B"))
 (segment (start 156.097001 98.777999) (end 153.975 100.9) (width 0.5) (layer "B.Cu") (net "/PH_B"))
 (segment (start 153.975 100.9) (end 144 100.9) (width 0.5) (layer "B.Cu") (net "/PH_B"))
 (segment (start 140.25 103.221934) (end 140.279524 103.251458) (width 0.5) (layer "B.Cu") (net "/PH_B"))
 (segment (start 143.175 100.075) (end 140.55 100.075) (width 0.5) (layer "B.Cu") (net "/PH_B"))
 (segment (start 158.637 98.59) (end 154.442433 102.784567) (width 0.5) (layer "B.Cu") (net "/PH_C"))
 (segment (start 154.442433 102.784567) (end 142.224264 102.784567) (width 0.5) (layer "B.Cu") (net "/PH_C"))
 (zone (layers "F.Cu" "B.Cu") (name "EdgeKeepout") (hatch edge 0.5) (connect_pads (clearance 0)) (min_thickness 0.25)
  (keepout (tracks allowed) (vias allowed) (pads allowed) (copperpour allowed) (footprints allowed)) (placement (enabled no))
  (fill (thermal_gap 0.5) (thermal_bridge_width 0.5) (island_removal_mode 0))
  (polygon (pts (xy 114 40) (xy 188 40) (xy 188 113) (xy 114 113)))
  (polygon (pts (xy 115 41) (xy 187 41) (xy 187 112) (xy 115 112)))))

